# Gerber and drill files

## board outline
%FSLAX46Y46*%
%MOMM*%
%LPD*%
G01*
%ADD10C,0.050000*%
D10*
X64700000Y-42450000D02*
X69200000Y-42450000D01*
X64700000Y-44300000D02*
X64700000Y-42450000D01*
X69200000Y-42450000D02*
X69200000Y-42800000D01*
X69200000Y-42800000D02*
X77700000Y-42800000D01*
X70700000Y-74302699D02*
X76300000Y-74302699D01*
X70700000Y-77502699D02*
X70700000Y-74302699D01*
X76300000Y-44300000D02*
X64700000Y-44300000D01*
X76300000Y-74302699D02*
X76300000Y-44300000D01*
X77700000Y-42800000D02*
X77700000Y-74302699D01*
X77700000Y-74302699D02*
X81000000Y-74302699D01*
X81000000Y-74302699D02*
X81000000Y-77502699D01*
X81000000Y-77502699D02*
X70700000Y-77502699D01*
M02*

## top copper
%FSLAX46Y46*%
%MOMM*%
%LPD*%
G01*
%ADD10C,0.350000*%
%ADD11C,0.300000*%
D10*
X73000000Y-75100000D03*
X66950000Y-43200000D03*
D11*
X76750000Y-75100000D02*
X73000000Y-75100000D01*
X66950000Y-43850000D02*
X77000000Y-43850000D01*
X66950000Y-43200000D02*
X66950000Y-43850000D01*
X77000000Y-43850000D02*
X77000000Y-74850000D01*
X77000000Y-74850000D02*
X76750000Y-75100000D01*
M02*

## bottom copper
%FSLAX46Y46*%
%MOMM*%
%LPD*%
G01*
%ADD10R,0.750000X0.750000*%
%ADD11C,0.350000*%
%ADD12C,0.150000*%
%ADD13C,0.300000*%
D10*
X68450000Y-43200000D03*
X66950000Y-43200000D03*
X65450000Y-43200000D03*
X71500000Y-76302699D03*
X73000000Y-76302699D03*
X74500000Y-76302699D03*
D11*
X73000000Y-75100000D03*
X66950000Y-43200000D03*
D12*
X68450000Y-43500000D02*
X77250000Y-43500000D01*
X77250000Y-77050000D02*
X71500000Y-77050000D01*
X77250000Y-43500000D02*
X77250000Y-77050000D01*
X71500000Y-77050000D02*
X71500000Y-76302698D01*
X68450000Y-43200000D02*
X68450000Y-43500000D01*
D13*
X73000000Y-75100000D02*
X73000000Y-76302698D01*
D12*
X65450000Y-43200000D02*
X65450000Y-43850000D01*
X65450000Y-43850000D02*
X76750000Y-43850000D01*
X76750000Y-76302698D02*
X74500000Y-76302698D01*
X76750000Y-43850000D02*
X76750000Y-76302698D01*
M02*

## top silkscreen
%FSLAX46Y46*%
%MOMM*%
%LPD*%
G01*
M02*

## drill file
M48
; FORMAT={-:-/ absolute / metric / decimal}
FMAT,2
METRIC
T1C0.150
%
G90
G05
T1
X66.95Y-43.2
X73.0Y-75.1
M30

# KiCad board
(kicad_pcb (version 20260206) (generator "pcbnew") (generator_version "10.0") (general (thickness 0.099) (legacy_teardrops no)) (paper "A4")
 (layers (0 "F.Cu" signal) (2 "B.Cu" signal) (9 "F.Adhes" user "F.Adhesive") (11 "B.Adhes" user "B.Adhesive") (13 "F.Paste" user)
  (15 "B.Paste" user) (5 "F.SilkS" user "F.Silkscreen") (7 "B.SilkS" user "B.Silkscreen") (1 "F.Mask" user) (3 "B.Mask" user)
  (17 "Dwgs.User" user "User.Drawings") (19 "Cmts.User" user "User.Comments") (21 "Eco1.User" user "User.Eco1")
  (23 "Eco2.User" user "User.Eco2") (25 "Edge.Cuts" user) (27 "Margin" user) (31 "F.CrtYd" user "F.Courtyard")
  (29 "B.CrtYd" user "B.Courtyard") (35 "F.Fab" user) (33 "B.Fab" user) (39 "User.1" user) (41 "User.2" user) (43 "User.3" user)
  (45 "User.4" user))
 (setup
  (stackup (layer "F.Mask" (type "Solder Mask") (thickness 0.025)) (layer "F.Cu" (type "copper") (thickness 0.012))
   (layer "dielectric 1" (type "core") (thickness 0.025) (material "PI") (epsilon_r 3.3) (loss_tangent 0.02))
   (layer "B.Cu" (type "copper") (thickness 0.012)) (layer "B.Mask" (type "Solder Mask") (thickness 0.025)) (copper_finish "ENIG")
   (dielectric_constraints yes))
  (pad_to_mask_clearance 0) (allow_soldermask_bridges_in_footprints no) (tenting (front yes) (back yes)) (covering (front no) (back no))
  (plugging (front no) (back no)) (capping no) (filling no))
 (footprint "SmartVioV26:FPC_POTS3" (layer "F.Cu") (at 0 0)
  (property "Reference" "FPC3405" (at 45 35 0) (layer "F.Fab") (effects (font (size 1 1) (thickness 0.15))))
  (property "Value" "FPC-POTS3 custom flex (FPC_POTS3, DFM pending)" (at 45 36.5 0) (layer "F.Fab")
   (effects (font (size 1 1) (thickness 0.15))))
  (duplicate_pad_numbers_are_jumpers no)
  (pad "S1" smd rect (at 68.45 43.2) (size 0.75 0.75) (layers "B.Cu" "B.Mask") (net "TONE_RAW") (solder_mask_margin 0.1))
  (pad "S2" smd rect (at 66.95 43.2) (size 0.75 0.75) (layers "B.Cu" "B.Mask") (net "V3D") (solder_mask_margin 0.1))
  (pad "S3" smd rect (at 65.45 43.2) (size 0.75 0.75) (layers "B.Cu" "B.Mask") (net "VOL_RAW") (solder_mask_margin 0.1))
  (pad "T1" smd rect (at 71.5 76.302699) (size 0.75 0.75) (layers "B.Cu" "B.Mask") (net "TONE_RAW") (solder_mask_margin 0.1))
  (pad "T2" smd rect (at 73 76.302699) (size 0.75 0.75) (layers "B.Cu" "B.Mask") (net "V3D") (solder_mask_margin 0.1))
  (pad "T3" smd rect (at 74.5 76.302699) (size 0.75 0.75) (layers "B.Cu" "B.Mask") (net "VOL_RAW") (solder_mask_margin 0.1)))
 (gr_line (start 64.7 42.45) (end 69.2 42.45) (stroke (width 0.05) (type default)) (layer "Edge.Cuts"))
 (gr_line (start 64.7 44.3) (end 64.7 42.45) (stroke (width 0.05) (type default)) (layer "Edge.Cuts"))
 (gr_line (start 69.2 42.45) (end 69.2 42.8) (stroke (width 0.05) (type default)) (layer "Edge.Cuts"))
 (gr_line (start 69.2 42.8) (end 77.7 42.8) (stroke (width 0.05) (type default)) (layer "Edge.Cuts"))
 (gr_line (start 70.7 74.302699) (end 76.3 74.302699) (stroke (width 0.05) (type default)) (layer "Edge.Cuts"))
 (gr_line (start 70.7 77.502699) (end 70.7 74.302699) (stroke (width 0.05) (type default)) (layer "Edge.Cuts"))
 (gr_line (start 76.3 44.3) (end 64.7 44.3) (stroke (width 0.05) (type default)) (layer "Edge.Cuts"))
 (gr_line (start 76.3 74.302699) (end 76.3 44.3) (stroke (width 0.05) (type default)) (layer "Edge.Cuts"))
 (gr_line (start 77.7 42.8) (end 77.7 74.302699) (stroke (width 0.05) (type default)) (layer "Edge.Cuts"))
 (gr_line (start 77.7 74.302699) (end 81 74.302699) (stroke (width 0.05) (type default)) (layer "Edge.Cuts"))
 (gr_line (start 81 74.302699) (end 81 77.502699) (stroke (width 0.05) (type default)) (layer "Edge.Cuts"))
 (gr_line (start 81 77.502699) (end 70.7 77.502699) (stroke (width 0.05) (type default)) (layer "Edge.Cuts"))
 (segment (start 68.45 43.5) (end 77.25 43.5) (width 0.15) (layer "B.Cu") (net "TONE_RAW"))
 (segment (start 77.25 77.05) (end 71.5 77.05) (width 0.15) (layer "B.Cu") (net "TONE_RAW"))
 (segment (start 77.25 43.5) (end 77.25 77.05) (width 0.15) (layer "B.Cu") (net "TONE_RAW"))
 (segment (start 71.5 77.05) (end 71.5 76.302698) (width 0.15) (layer "B.Cu") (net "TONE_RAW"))
 (segment (start 68.45 43.2) (end 68.45 43.5) (width 0.15) (layer "B.Cu") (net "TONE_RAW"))
 (segment (start 76.75 75.1) (end 73 75.1) (width 0.3) (layer "F.Cu") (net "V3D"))
 (segment (start 66.95 43.85) (end 77 43.85) (width 0.3) (layer "F.Cu") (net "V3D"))
 (segment (start 66.95 43.2) (end 66.95 43.85) (width 0.3) (layer "F.Cu") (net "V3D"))
 (segment (start 77 43.85) (end 77 74.85) (width 0.3) (layer "F.Cu") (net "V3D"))
 (segment (start 77 74.85) (end 76.75 75.1) (width 0.3) (layer "F.Cu") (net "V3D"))
 (via (at 73 75.1) (size 0.35) (drill 0.15) (layers "F.Cu" "B.Cu") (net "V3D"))
 (via (at 66.95 43.2) (size 0.35) (drill 0.15) (layers "F.Cu" "B.Cu") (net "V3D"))
 (segment (start 73 75.1) (end 73 76.302698) (width 0.3) (layer "B.Cu") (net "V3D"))
 (segment (start 65.45 43.2) (end 65.45 43.85) (width 0.15) (layer "B.Cu") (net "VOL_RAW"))
 (segment (start 65.45 43.85) (end 76.75 43.85) (width 0.15) (layer "B.Cu") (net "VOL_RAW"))
 (segment (start 76.75 76.302698) (end 74.5 76.302698) (width 0.15) (layer "B.Cu") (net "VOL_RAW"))
 (segment (start 76.75 43.85) (end 76.75 76.302698) (width 0.15) (layer "B.Cu") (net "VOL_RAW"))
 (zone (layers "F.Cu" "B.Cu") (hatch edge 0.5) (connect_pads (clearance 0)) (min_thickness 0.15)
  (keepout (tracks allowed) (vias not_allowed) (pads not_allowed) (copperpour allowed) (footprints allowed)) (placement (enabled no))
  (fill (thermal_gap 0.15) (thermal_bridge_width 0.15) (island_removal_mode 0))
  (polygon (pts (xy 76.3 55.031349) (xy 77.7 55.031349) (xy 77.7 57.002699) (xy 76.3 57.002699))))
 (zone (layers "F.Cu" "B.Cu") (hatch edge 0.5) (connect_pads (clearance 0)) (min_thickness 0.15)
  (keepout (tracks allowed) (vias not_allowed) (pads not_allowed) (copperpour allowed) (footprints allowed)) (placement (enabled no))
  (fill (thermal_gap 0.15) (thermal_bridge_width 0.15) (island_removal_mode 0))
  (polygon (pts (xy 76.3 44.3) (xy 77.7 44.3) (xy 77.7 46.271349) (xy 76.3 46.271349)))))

